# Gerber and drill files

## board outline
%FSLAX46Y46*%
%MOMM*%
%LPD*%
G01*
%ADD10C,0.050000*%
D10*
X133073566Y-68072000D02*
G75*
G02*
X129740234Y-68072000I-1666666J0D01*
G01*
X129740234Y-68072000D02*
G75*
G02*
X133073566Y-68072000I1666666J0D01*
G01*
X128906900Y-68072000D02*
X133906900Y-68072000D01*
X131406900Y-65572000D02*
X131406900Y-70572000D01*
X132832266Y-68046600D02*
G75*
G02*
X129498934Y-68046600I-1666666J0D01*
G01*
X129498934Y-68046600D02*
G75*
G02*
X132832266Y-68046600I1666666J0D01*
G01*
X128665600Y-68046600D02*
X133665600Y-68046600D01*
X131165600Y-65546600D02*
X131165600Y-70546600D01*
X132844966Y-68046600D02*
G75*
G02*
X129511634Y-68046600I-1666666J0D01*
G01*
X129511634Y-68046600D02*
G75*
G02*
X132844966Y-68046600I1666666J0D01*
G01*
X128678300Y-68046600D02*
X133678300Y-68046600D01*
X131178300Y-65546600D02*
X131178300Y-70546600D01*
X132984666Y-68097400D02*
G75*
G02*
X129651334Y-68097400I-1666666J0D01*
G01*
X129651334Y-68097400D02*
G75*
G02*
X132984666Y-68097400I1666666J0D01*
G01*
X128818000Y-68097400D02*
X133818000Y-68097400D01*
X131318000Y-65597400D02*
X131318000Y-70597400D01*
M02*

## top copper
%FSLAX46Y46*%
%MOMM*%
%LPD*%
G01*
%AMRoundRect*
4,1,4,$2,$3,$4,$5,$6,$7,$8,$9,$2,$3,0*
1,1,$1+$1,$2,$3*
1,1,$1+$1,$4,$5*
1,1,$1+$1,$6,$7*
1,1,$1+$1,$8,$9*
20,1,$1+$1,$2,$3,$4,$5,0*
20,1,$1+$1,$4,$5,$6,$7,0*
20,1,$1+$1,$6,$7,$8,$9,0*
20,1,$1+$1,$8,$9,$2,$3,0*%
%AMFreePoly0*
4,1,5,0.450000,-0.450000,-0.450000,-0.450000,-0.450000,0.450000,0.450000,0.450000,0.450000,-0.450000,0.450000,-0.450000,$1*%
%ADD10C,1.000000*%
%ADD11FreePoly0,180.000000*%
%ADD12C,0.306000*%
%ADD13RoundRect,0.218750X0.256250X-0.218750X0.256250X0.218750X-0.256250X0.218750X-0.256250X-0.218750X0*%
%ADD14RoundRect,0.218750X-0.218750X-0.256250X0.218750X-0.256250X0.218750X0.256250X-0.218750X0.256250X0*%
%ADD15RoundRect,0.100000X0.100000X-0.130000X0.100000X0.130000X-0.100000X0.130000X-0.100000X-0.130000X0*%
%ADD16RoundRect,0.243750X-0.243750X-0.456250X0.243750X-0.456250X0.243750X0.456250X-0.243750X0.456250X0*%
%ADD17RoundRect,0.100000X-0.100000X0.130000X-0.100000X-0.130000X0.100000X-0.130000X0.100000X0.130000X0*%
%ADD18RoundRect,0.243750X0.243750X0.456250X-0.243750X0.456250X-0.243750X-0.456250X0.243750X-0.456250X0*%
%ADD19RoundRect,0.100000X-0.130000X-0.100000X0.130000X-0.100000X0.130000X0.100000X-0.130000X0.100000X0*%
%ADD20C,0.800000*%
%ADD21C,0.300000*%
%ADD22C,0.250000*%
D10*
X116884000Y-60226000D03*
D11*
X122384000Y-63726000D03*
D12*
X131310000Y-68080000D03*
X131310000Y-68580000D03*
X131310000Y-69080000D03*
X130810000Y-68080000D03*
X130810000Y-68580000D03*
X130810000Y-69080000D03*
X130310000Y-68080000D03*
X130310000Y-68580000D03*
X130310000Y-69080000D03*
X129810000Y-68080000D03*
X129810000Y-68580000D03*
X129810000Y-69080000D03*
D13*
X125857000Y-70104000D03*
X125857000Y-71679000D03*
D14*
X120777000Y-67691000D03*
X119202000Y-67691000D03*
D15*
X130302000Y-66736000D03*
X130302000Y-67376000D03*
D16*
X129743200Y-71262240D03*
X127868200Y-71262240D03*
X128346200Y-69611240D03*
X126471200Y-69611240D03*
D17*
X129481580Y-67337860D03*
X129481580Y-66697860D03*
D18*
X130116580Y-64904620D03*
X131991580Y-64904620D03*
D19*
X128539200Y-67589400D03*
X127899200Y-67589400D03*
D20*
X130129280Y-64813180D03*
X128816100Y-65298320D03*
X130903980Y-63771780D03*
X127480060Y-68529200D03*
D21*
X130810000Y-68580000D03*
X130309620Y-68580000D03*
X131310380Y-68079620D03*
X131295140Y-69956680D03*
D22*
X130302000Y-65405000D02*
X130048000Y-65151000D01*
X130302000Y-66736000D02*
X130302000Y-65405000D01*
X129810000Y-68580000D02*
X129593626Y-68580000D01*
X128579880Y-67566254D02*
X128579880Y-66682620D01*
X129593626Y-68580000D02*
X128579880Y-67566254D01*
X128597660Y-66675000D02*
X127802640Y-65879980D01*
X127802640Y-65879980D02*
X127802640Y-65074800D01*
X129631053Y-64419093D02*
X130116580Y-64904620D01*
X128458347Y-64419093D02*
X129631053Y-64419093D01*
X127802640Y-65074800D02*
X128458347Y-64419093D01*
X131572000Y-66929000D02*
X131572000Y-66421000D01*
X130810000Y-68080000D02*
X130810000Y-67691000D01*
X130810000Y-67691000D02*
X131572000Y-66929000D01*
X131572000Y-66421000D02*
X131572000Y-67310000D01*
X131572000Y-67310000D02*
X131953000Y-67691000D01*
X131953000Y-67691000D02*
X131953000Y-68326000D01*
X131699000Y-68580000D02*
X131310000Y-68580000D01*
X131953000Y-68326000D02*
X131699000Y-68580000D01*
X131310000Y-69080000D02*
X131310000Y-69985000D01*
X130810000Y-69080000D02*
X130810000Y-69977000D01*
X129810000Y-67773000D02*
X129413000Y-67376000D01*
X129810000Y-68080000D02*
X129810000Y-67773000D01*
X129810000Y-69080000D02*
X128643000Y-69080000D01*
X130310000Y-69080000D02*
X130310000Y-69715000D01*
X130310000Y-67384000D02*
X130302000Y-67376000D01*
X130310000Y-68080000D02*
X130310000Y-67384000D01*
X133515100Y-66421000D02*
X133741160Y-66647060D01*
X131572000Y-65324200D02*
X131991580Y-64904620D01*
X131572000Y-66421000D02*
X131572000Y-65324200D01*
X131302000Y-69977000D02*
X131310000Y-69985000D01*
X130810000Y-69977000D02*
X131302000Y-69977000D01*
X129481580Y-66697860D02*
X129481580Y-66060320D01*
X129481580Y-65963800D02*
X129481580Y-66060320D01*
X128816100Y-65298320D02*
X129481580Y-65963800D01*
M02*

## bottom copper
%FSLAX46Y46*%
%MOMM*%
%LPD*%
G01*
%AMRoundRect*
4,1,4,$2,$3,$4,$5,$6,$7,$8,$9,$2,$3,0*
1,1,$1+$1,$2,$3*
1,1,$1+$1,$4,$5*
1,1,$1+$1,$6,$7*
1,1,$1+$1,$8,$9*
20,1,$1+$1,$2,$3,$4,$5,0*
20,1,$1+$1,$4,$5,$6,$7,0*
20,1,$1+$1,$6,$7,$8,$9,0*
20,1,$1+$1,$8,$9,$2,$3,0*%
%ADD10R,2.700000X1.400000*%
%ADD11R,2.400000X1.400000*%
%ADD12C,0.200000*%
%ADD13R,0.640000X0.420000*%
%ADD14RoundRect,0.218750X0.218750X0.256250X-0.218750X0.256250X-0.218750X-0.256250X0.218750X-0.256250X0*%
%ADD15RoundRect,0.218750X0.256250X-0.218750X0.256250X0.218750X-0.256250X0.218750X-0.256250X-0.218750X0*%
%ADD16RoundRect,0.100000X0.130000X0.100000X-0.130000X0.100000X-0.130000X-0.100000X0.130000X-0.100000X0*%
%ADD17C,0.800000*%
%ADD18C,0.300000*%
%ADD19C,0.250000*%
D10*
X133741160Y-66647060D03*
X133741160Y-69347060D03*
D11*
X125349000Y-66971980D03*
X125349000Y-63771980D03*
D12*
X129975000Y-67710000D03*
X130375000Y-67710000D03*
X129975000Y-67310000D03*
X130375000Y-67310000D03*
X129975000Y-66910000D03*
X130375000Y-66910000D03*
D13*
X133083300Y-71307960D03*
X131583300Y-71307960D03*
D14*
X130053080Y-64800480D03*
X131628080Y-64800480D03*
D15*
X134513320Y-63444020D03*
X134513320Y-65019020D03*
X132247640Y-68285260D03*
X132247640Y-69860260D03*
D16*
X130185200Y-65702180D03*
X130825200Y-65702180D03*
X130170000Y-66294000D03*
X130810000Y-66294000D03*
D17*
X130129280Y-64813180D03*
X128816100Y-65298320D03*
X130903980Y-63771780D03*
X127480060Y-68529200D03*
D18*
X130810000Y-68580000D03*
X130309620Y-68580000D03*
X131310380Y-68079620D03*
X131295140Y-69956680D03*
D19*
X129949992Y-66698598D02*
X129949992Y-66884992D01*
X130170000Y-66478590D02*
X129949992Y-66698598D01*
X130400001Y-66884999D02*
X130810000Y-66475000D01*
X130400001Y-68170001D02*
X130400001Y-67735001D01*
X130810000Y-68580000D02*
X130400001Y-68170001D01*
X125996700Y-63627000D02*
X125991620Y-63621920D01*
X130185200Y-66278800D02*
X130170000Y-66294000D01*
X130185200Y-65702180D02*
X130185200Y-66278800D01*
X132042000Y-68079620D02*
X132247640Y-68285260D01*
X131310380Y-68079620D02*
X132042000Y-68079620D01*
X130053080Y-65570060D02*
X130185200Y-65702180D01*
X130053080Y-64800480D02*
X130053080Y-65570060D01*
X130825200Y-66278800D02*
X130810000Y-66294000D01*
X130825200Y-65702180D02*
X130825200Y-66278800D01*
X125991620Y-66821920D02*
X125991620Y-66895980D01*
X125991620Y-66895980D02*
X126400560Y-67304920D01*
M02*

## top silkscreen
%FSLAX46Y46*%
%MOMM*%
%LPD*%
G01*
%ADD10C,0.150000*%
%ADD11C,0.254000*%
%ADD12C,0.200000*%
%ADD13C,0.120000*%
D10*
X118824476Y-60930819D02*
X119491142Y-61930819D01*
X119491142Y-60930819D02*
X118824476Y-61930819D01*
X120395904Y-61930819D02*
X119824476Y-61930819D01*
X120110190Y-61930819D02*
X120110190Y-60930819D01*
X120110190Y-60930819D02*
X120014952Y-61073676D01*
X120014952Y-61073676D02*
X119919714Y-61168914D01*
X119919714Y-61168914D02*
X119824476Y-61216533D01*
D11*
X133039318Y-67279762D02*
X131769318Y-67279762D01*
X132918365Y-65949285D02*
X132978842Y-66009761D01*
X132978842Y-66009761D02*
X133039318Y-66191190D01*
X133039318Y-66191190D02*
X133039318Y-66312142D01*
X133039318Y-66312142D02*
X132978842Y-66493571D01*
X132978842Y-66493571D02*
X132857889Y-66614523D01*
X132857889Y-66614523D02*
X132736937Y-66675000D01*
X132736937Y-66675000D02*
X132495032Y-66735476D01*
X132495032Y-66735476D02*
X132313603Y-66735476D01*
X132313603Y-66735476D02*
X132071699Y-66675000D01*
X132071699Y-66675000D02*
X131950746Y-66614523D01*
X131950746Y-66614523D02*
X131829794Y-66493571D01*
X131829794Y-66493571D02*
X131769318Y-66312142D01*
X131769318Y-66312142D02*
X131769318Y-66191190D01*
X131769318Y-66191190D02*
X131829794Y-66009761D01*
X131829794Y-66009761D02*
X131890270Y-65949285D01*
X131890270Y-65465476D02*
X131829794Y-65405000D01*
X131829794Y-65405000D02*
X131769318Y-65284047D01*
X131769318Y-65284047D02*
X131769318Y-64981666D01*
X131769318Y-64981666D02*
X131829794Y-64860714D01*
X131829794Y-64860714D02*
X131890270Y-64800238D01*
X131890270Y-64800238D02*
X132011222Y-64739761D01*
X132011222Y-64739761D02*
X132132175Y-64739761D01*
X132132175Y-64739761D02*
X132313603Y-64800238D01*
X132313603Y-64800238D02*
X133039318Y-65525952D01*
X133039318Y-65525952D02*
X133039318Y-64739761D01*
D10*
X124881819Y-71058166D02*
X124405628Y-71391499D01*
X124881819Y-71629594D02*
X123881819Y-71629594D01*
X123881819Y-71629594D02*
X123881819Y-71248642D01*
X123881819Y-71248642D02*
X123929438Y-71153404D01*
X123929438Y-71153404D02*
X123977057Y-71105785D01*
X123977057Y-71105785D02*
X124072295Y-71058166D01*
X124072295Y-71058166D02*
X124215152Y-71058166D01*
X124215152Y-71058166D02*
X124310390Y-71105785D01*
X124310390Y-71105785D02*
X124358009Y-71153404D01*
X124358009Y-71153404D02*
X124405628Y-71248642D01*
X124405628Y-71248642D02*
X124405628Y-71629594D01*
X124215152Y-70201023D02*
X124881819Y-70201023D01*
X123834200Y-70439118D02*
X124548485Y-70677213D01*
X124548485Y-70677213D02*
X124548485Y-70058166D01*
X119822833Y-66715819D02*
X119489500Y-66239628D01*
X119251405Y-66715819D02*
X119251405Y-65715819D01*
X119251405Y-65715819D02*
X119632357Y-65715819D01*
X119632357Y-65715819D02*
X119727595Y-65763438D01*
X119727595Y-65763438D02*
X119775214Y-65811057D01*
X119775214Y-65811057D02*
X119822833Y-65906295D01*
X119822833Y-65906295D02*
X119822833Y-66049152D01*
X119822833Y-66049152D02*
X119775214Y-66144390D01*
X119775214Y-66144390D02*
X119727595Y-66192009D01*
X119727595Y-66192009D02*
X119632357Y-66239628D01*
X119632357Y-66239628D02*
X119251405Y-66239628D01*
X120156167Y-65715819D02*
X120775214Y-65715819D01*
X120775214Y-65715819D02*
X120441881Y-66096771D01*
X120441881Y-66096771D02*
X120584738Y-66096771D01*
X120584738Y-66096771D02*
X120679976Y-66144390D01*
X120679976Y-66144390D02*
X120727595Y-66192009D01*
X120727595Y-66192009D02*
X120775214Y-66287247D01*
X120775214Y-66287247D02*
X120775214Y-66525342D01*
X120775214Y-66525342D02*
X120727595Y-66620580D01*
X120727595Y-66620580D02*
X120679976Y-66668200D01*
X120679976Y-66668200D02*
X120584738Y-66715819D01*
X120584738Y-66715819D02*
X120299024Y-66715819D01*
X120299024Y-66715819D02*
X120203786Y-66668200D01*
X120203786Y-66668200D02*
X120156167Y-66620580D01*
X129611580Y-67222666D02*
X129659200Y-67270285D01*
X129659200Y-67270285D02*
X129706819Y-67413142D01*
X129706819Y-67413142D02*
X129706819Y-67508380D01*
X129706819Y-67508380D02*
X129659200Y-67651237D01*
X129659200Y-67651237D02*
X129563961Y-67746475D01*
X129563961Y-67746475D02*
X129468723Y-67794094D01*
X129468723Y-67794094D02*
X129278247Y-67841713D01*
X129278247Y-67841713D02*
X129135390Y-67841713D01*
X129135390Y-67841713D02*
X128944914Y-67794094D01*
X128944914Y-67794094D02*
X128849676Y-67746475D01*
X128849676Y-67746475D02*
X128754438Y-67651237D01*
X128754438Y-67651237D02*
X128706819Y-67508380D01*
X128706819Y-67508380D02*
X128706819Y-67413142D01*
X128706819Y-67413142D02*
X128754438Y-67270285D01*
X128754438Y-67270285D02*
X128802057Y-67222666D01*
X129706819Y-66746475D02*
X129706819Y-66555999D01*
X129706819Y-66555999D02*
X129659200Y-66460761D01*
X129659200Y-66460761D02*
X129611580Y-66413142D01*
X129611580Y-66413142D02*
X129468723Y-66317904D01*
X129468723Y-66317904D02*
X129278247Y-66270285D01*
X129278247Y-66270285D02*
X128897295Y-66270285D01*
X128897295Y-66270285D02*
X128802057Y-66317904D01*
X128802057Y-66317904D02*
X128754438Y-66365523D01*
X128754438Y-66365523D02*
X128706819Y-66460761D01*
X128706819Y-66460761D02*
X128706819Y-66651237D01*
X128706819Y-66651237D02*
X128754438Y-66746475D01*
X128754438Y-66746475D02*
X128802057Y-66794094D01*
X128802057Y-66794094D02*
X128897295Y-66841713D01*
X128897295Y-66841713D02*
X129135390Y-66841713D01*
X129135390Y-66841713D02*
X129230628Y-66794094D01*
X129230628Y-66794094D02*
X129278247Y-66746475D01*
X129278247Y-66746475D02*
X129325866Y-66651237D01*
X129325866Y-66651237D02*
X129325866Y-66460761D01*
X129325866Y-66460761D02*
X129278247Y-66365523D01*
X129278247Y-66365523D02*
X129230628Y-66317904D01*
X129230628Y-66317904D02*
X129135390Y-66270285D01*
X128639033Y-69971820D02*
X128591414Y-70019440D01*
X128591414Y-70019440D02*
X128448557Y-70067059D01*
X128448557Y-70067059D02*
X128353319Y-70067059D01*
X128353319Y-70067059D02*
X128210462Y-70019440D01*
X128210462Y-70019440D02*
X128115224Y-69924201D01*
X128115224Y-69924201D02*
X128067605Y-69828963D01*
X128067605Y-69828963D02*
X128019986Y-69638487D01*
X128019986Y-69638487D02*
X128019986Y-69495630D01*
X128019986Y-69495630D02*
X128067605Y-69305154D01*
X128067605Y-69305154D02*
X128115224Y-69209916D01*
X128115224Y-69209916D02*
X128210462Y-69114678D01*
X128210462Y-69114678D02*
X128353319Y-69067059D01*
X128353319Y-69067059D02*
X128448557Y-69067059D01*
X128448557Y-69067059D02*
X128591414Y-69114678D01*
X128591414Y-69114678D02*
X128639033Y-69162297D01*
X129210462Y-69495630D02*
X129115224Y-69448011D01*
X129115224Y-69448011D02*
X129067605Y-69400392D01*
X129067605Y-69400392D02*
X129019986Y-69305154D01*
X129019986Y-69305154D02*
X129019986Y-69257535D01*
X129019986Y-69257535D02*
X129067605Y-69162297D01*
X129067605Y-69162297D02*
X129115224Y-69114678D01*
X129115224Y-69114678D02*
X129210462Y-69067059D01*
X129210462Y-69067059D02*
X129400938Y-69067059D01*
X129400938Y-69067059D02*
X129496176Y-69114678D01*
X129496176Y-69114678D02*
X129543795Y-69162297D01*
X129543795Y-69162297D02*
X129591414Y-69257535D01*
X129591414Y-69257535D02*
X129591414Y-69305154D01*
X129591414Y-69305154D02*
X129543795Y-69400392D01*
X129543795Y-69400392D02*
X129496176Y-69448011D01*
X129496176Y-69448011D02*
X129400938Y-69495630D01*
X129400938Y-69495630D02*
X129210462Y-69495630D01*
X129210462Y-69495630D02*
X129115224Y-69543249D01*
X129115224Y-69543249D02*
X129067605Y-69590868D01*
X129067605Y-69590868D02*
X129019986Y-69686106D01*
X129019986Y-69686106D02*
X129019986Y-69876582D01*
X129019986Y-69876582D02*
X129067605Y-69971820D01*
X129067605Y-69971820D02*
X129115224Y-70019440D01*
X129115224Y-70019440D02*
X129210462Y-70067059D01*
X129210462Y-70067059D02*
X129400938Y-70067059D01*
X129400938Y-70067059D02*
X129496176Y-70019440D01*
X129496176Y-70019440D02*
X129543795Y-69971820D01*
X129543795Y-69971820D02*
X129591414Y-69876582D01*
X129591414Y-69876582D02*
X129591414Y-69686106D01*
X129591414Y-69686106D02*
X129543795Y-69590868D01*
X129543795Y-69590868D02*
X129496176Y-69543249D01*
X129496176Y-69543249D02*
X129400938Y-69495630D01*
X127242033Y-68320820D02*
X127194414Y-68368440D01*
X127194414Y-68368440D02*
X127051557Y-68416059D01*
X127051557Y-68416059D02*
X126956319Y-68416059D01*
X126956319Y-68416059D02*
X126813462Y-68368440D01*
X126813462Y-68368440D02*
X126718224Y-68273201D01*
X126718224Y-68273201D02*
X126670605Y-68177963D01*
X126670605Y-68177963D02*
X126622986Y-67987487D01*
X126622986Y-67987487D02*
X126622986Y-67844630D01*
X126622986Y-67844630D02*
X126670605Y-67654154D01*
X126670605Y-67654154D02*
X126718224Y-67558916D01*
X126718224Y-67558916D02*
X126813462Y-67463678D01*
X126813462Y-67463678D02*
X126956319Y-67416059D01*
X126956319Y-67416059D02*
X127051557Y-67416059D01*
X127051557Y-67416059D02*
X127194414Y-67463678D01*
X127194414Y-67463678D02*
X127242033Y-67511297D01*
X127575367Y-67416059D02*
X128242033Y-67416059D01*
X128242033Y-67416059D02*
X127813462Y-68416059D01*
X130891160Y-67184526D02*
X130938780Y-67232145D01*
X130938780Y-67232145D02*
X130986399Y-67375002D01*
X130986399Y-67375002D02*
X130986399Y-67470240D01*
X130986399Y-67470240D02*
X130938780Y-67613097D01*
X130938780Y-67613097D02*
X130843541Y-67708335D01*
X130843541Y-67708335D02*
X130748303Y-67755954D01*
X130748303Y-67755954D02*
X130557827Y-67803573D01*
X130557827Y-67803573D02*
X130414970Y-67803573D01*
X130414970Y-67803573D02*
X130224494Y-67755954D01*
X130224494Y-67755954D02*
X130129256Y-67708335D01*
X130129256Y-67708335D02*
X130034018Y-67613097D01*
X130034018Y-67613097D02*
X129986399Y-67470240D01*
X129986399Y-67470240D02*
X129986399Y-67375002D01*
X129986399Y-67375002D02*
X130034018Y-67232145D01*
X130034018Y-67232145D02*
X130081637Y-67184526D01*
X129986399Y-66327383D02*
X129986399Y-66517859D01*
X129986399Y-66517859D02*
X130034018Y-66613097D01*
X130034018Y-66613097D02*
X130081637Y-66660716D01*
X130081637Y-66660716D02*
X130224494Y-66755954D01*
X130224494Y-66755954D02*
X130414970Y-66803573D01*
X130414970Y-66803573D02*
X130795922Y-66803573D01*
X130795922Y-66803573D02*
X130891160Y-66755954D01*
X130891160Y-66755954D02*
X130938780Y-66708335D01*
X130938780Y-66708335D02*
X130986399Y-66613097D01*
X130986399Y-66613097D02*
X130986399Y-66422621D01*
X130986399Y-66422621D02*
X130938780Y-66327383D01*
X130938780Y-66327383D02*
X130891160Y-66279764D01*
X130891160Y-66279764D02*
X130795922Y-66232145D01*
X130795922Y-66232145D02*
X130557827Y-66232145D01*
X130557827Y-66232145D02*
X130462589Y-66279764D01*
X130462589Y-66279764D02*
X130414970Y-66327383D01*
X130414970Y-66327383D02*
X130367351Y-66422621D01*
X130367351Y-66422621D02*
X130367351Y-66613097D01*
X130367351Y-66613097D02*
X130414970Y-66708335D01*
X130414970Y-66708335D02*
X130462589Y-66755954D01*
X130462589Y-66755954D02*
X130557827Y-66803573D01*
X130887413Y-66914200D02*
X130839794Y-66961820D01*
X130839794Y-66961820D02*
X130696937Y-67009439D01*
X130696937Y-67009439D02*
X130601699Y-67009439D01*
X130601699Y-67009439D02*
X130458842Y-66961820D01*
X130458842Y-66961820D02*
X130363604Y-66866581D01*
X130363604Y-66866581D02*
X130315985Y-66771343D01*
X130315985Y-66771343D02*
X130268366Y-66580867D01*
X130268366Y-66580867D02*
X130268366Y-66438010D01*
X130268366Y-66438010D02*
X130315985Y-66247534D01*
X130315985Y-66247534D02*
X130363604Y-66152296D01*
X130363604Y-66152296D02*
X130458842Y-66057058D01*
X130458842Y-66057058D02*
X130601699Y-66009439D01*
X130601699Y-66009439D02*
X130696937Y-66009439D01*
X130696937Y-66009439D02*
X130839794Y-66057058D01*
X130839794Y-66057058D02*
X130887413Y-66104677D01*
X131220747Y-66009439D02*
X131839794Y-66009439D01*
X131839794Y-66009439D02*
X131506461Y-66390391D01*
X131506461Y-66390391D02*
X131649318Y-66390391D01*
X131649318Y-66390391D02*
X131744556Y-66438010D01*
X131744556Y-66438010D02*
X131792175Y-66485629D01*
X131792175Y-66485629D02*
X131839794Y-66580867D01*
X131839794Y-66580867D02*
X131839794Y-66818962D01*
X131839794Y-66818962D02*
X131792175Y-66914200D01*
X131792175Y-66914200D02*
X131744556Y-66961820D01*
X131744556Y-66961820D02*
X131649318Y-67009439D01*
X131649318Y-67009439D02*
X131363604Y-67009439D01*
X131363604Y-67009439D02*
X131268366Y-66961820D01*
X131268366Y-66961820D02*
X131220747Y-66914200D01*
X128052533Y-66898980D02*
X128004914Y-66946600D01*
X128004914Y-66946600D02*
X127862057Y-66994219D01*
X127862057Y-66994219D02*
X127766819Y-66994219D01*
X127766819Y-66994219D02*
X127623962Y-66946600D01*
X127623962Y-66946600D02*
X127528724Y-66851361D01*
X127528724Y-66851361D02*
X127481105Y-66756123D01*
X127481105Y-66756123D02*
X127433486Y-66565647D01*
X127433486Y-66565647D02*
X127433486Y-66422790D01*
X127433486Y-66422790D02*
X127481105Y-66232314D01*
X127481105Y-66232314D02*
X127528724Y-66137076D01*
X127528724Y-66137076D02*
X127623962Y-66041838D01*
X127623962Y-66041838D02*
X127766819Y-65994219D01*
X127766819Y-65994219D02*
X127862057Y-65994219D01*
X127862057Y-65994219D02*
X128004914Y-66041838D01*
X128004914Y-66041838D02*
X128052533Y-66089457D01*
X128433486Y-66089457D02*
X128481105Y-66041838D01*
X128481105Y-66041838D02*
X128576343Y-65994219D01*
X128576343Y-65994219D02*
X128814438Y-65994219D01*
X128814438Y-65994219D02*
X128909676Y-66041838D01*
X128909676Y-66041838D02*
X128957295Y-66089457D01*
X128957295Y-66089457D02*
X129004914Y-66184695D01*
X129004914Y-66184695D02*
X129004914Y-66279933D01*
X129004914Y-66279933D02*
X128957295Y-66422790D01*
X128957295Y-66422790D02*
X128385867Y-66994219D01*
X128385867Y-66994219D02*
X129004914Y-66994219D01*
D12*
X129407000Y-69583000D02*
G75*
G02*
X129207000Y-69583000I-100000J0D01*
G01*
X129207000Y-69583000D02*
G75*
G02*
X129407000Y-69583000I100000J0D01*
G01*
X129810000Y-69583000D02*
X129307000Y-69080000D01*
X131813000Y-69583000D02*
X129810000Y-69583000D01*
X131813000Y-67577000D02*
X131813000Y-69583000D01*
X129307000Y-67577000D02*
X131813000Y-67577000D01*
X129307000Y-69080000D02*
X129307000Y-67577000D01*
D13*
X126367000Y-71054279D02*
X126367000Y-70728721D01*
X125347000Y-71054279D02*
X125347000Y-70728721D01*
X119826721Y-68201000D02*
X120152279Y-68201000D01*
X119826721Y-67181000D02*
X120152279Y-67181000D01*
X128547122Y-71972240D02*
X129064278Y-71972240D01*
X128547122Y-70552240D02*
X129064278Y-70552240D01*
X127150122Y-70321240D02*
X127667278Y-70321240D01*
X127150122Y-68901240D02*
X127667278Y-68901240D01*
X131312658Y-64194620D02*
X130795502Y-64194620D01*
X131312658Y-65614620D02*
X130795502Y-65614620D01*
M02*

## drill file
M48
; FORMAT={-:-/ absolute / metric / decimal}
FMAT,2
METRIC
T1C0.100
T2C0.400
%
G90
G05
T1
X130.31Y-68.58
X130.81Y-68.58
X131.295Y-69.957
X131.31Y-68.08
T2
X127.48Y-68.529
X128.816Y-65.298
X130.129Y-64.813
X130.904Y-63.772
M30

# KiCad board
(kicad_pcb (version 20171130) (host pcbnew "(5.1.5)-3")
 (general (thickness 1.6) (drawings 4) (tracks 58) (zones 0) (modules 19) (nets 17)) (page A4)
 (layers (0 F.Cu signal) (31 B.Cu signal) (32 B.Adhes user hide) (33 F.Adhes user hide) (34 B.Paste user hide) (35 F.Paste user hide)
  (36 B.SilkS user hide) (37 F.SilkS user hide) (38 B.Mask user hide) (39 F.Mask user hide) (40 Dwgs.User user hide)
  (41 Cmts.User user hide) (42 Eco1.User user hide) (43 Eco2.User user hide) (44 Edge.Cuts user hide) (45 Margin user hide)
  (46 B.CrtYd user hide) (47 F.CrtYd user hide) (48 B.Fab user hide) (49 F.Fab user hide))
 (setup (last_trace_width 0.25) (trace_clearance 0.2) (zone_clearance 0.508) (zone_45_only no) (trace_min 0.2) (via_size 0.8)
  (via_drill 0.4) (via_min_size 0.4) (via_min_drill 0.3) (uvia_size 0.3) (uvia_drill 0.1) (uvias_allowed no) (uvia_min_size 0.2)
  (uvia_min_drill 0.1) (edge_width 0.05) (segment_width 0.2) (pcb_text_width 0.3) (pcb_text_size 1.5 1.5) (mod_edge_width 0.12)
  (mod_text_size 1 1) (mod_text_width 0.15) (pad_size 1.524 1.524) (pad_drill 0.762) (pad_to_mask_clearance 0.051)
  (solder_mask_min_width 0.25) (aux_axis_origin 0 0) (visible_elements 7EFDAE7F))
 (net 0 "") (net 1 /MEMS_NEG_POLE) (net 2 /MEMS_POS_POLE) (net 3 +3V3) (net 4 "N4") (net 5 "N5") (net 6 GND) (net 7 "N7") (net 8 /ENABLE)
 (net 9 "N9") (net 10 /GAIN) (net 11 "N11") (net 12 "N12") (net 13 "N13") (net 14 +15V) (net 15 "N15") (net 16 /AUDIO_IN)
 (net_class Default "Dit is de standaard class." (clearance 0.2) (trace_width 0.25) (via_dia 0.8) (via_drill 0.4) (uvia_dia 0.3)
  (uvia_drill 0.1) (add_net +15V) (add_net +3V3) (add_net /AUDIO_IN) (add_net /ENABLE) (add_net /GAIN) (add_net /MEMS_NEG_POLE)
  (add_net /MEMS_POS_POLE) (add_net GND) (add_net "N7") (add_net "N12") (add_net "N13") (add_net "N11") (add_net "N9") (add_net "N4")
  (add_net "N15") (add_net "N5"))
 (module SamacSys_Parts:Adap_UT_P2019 (layer F.Cu) (at 119.634 61.976 180) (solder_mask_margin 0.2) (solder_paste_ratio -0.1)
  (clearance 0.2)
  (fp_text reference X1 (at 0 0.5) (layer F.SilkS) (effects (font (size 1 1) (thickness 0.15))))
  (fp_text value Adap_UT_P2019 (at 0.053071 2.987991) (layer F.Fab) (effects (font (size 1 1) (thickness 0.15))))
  (pad 2 smd circle (at 2.75 1.75 180) (size 1 1) (layers F.Cu F.Paste F.Mask) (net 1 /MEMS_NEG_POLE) (zone_connect 0))
  (pad 1 smd custom (at -2.75 -1.75 180) (size 0.9 0.9) (layers F.Cu F.Paste F.Mask) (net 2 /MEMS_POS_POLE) (zone_connect 0)
   (options (clearance outline) (anchor rect)) (primitives)))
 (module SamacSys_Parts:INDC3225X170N (layer B.Cu) (at 133.74116 67.99706 90)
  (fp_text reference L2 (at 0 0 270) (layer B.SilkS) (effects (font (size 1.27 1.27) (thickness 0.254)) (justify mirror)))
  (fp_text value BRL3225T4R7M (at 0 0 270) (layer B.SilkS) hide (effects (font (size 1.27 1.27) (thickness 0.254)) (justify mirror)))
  (pad 2 smd rect (at 1.35 0 90) (size 1.4 2.7) (layers B.Cu B.Paste B.Mask) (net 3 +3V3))
  (pad 1 smd rect (at -1.35 0 90) (size 1.4 2.7) (layers B.Cu B.Paste B.Mask) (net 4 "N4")))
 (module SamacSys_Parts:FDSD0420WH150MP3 (layer B.Cu) (at 125.349 65.37198 270)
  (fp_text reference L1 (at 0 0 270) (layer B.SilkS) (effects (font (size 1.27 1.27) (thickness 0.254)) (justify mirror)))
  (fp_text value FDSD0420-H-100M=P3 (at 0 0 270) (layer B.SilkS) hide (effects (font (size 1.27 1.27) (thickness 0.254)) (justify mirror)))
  (pad 2 smd rect (at 1.6 0 270) (size 1.4 2.4) (layers B.Cu B.Paste B.Mask) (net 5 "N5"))
  (pad 1 smd rect (at -1.6 0 270) (size 1.4 2.4) (layers B.Cu B.Paste B.Mask) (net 3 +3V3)))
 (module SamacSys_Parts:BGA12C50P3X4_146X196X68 (layer F.Cu) (at 130.56 68.58 90)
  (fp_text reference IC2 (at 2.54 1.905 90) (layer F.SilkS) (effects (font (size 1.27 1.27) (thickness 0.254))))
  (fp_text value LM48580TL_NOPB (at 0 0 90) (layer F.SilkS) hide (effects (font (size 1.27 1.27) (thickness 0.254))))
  (fp_circle (center -1.003 -1.253) (end -1.003 -1.153) (layer F.SilkS) (width 0.2))
  (fp_line (start -1.003 -0.75) (end -0.5 -1.253) (layer F.SilkS) (width 0.2))
  (fp_line (start -1.003 1.253) (end -1.003 -0.75) (layer F.SilkS) (width 0.2))
  (fp_line (start 1.003 1.253) (end -1.003 1.253) (layer F.SilkS) (width 0.2))
  (fp_line (start 1.003 -1.253) (end 1.003 1.253) (layer F.SilkS) (width 0.2))
  (fp_line (start -0.5 -1.253) (end 1.003 -1.253) (layer F.SilkS) (width 0.2))
  (pad D3 smd circle (at 0.5 0.75 180) (size 0.306 0.306) (layers F.Cu F.Paste F.Mask) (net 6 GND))
  (pad D2 smd circle (at 0 0.75 180) (size 0.306 0.306) (layers F.Cu F.Paste F.Mask) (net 3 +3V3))
  (pad D1 smd circle (at -0.5 0.75 180) (size 0.306 0.306) (layers F.Cu F.Paste F.Mask) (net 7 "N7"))
  (pad C3 smd circle (at 0.5 0.25 180) (size 0.306 0.306) (layers F.Cu F.Paste F.Mask) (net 3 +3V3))
  (pad C2 smd circle (at 0 0.25 180) (size 0.306 0.306) (layers F.Cu F.Paste F.Mask) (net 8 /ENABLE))
  (pad C1 smd circle (at -0.5 0.25 180) (size 0.306 0.306) (layers F.Cu F.Paste F.Mask) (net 7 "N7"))
  (pad B3 smd circle (at 0.5 -0.25 180) (size 0.306 0.306) (layers F.Cu F.Paste F.Mask) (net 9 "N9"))
  (pad B2 smd circle (at 0 -0.25 180) (size 0.306 0.306) (layers F.Cu F.Paste F.Mask) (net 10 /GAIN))
  (pad B1 smd circle (at -0.5 -0.25 180) (size 0.306 0.306) (layers F.Cu F.Paste F.Mask) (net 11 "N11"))
  (pad A3 smd circle (at 0.5 -0.75 180) (size 0.306 0.306) (layers F.Cu F.Paste F.Mask) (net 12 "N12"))
  (pad A2 smd circle (at 0 -0.75 180) (size 0.306 0.306) (layers F.Cu F.Paste F.Mask) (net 6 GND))
  (pad A1 smd circle (at -0.5 -0.75 180) (size 0.306 0.306) (layers F.Cu F.Paste F.Mask) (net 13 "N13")))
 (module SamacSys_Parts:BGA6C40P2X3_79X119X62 (layer B.Cu) (at 130.175 67.31 180)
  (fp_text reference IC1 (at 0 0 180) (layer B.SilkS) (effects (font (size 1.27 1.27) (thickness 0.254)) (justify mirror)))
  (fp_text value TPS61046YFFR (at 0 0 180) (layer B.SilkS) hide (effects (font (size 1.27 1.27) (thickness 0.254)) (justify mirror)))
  (pad C2 smd circle (at 0.2 -0.4 90) (size 0.2 0.2) (layers B.Cu B.Paste B.Mask) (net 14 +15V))
  (pad C1 smd circle (at -0.2 -0.4 90) (size 0.2 0.2) (layers B.Cu B.Paste B.Mask) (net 8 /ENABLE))
  (pad B2 smd circle (at 0.2 0 90) (size 0.2 0.2) (layers B.Cu B.Paste B.Mask) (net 5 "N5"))
  (pad B1 smd circle (at -0.2 0 90) (size 0.2 0.2) (layers B.Cu B.Paste B.Mask) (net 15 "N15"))
  (pad A2 smd circle (at 0.2 0.4 90) (size 0.2 0.2) (layers B.Cu B.Paste B.Mask) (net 6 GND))
  (pad A1 smd circle (at -0.2 0.4 90) (size 0.2 0.2) (layers B.Cu B.Paste B.Mask) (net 3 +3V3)))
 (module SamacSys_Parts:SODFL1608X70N (layer B.Cu) (at 132.3333 71.30796)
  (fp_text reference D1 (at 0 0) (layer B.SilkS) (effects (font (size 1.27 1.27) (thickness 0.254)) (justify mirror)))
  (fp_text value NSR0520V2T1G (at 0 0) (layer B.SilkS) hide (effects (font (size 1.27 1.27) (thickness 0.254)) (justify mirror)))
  (pad 2 smd rect (at 0.75 0 270) (size 0.42 0.64) (layers B.Cu B.Paste B.Mask) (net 4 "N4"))
  (pad 1 smd rect (at -0.75 0 270) (size 0.42 0.64) (layers B.Cu B.Paste B.Mask) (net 7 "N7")))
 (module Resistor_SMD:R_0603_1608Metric (layer F.Cu) (at 125.857 70.8915 90)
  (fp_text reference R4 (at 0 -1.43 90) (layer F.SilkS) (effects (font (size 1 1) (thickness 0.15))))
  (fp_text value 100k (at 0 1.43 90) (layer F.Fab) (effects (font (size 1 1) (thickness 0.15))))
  (fp_line (start -0.162779 0.51) (end 0.162779 0.51) (layer F.SilkS) (width 0.12))
  (fp_line (start -0.162779 -0.51) (end 0.162779 -0.51) (layer F.SilkS) (width 0.12))
  (pad 2 smd roundrect (at 0.7875 0 90) (size 0.875 0.95) (layers F.Cu F.Paste F.Mask) (roundrect_rratio 0.25) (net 14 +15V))
  (pad 1 smd roundrect (at -0.7875 0 90) (size 0.875 0.95) (layers F.Cu F.Paste F.Mask) (roundrect_rratio 0.25) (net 1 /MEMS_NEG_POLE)))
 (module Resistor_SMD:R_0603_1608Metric (layer F.Cu) (at 119.9895 67.691)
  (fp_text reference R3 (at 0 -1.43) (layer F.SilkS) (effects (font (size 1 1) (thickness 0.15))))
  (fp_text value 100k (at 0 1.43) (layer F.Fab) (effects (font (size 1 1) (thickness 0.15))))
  (fp_line (start -0.162779 0.51) (end 0.162779 0.51) (layer F.SilkS) (width 0.12))
  (fp_line (start -0.162779 -0.51) (end 0.162779 -0.51) (layer F.SilkS) (width 0.12))
  (pad 2 smd roundrect (at 0.7875 0) (size 0.875 0.95) (layers F.Cu F.Paste F.Mask) (roundrect_rratio 0.25) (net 14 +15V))
  (pad 1 smd roundrect (at -0.7875 0) (size 0.875 0.95) (layers F.Cu F.Paste F.Mask) (roundrect_rratio 0.25) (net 2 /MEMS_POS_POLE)))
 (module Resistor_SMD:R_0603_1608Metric (layer B.Cu) (at 130.84058 64.80048 180)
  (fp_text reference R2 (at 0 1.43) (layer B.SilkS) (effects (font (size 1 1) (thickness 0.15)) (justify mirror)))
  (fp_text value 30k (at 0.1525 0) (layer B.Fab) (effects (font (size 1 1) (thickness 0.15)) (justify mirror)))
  (pad 2 smd roundrect (at 0.7875 0 180) (size 0.875 0.95) (layers B.Cu B.Paste B.Mask) (roundrect_rratio 0.25) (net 6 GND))
  (pad 1 smd roundrect (at -0.7875 0 180) (size 0.875 0.95) (layers B.Cu B.Paste B.Mask) (roundrect_rratio 0.25) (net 15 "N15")))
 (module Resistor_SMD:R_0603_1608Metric (layer B.Cu) (at 134.51332 64.23152 90)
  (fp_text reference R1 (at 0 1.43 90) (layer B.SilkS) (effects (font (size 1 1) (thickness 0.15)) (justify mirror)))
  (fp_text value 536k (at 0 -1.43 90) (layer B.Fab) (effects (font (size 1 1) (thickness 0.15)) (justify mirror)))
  (pad 2 smd roundrect (at 0.7875 0 90) (size 0.875 0.95) (layers B.Cu B.Paste B.Mask) (roundrect_rratio 0.25) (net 15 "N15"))
  (pad 1 smd roundrect (at -0.7875 0 90) (size 0.875 0.95) (layers B.Cu B.Paste B.Mask) (roundrect_rratio 0.25) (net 14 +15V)))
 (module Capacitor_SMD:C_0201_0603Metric (layer F.Cu) (at 130.302 67.056 90)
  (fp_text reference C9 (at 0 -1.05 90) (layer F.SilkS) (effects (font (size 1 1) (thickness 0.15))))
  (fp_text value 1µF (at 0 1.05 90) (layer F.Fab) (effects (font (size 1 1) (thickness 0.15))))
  (pad 2 smd roundrect (at 0.32 0 90) (size 0.46 0.4) (layers F.Cu F.Mask) (roundrect_rratio 0.25) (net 6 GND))
  (pad 1 smd roundrect (at -0.32 0 90) (size 0.46 0.4) (layers F.Cu F.Mask) (roundrect_rratio 0.25) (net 9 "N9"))
  (pad "" smd roundrect (at 0.345 0 90) (size 0.318 0.36) (layers F.Paste) (roundrect_rratio 0.25))
  (pad "" smd roundrect (at -0.345 0 90) (size 0.318 0.36) (layers F.Paste) (roundrect_rratio 0.25)))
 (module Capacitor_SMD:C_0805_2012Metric (layer F.Cu) (at 128.8057 71.26224)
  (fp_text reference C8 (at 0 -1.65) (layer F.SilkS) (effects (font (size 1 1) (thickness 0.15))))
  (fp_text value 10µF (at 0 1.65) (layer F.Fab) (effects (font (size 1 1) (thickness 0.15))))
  (fp_line (start -0.258578 0.71) (end 0.258578 0.71) (layer F.SilkS) (width 0.12))
  (fp_line (start -0.258578 -0.71) (end 0.258578 -0.71) (layer F.SilkS) (width 0.12))
  (pad 2 smd roundrect (at 0.9375 0) (size 0.975 1.4) (layers F.Cu F.Paste F.Mask) (roundrect_rratio 0.25) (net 11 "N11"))
  (pad 1 smd roundrect (at -0.9375 0) (size 0.975 1.4) (layers F.Cu F.Paste F.Mask) (roundrect_rratio 0.25) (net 1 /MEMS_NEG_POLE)))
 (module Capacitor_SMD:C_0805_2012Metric (layer F.Cu) (at 127.4087 69.61124)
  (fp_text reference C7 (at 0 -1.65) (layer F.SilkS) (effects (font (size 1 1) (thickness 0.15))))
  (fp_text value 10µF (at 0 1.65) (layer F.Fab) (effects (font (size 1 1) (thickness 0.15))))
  (fp_line (start -0.258578 0.71) (end 0.258578 0.71) (layer F.SilkS) (width 0.12))
  (fp_line (start -0.258578 -0.71) (end 0.258578 -0.71) (layer F.SilkS) (width 0.12))
  (pad 2 smd roundrect (at 0.9375 0) (size 0.975 1.4) (layers F.Cu F.Paste F.Mask) (roundrect_rratio 0.25) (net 13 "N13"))
  (pad 1 smd roundrect (at -0.9375 0) (size 0.975 1.4) (layers F.Cu F.Paste F.Mask) (roundrect_rratio 0.25) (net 2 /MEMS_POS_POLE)))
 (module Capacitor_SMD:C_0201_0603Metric (layer F.Cu) (at 129.48158 67.01786 270)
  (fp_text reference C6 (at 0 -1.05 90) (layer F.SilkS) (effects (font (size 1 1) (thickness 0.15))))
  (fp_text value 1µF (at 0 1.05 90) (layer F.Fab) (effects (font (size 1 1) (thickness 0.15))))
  (pad 2 smd roundrect (at 0.32 0 270) (size 0.46 0.4) (layers F.Cu F.Mask) (roundrect_rratio 0.25) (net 12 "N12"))
  (pad 1 smd roundrect (at -0.32 0 270) (size 0.46 0.4) (layers F.Cu F.Mask) (roundrect_rratio 0.25) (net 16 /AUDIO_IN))
  (pad "" smd roundrect (at 0.345 0 270) (size 0.318 0.36) (layers F.Paste) (roundrect_rratio 0.25))
  (pad "" smd roundrect (at -0.345 0 270) (size 0.318 0.36) (layers F.Paste) (roundrect_rratio 0.25)))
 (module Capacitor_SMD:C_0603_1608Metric (layer B.Cu) (at 132.24764 69.07276 90)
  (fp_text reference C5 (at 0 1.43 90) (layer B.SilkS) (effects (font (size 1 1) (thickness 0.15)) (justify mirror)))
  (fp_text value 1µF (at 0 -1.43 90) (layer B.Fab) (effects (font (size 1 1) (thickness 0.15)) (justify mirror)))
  (pad 2 smd roundrect (at 0.7875 0 90) (size 0.875 0.95) (layers B.Cu B.Paste B.Mask) (roundrect_rratio 0.25) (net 6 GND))
  (pad 1 smd roundrect (at -0.7875 0 90) (size 0.875 0.95) (layers B.Cu B.Paste B.Mask) (roundrect_rratio 0.25) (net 7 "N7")))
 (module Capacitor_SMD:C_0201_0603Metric (layer B.Cu) (at 130.5052 65.70218 180)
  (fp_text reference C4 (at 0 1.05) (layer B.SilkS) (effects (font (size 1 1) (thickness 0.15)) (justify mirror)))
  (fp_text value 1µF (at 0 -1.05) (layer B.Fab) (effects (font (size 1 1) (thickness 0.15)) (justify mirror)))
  (pad 2 smd roundrect (at 0.32 0 180) (size 0.46 0.4) (layers B.Cu B.Mask) (roundrect_rratio 0.25) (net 6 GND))
  (pad 1 smd roundrect (at -0.32 0 180) (size 0.46 0.4) (layers B.Cu B.Mask) (roundrect_rratio 0.25) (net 3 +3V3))
  (pad "" smd roundrect (at 0.345 0 180) (size 0.318 0.36) (layers B.Paste) (roundrect_rratio 0.25))
  (pad "" smd roundrect (at -0.345 0 180) (size 0.318 0.36) (layers B.Paste) (roundrect_rratio 0.25)))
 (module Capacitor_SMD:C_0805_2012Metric (layer F.Cu) (at 131.05408 64.90462 180)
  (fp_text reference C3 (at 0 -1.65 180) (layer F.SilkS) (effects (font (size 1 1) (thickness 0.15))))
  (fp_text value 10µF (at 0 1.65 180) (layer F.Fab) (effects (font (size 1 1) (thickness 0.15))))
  (fp_line (start -0.258578 0.71) (end 0.258578 0.71) (layer F.SilkS) (width 0.12))
  (fp_line (start -0.258578 -0.71) (end 0.258578 -0.71) (layer F.SilkS) (width 0.12))
  (pad 2 smd roundrect (at 0.9375 0 180) (size 0.975 1.4) (layers F.Cu F.Paste F.Mask) (roundrect_rratio 0.25) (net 6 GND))
  (pad 1 smd roundrect (at -0.9375 0 180) (size 0.975 1.4) (layers F.Cu F.Paste F.Mask) (roundrect_rratio 0.25) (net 3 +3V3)))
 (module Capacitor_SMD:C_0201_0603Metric (layer F.Cu) (at 128.2192 67.5894)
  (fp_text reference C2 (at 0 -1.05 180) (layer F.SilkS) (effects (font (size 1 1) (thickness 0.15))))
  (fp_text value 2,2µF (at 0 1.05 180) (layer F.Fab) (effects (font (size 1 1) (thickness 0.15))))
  (pad 2 smd roundrect (at 0.32 0) (size 0.46 0.4) (layers F.Cu F.Mask) (roundrect_rratio 0.25) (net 6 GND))
  (pad 1 smd roundrect (at -0.32 0) (size 0.46 0.4) (layers F.Cu F.Mask) (roundrect_rratio 0.25) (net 14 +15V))
  (pad "" smd roundrect (at 0.345 0) (size 0.318 0.36) (layers F.Paste) (roundrect_rratio 0.25))
  (pad "" smd roundrect (at -0.345 0) (size 0.318 0.36) (layers F.Paste) (roundrect_rratio 0.25)))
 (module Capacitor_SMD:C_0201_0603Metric (layer B.Cu) (at 130.49 66.294 180)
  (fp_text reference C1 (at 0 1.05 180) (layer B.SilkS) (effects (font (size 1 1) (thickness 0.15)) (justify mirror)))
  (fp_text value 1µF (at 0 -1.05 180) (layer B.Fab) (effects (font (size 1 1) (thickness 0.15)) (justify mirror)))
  (pad 2 smd roundrect (at 0.32 0 180) (size 0.46 0.4) (layers B.Cu B.Mask) (roundrect_rratio 0.25) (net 6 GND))
  (pad 1 smd roundrect (at -0.32 0 180) (size 0.46 0.4) (layers B.Cu B.Mask) (roundrect_rratio 0.25) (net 3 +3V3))
  (pad "" smd roundrect (at 0.345 0 180) (size 0.318 0.36) (layers B.Paste) (roundrect_rratio 0.25))
  (pad "" smd roundrect (at -0.345 0 180) (size 0.318 0.36) (layers B.Paste) (roundrect_rratio 0.25)))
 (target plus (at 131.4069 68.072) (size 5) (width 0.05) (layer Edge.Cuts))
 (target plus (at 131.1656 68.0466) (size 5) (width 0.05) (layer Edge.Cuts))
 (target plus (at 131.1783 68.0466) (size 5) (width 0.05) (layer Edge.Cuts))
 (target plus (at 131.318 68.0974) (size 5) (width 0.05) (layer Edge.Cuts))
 (via (at 130.12928 64.81318) (size 0.8) (drill 0.4) (layers F.Cu B.Cu) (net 6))
 (segment (start 130.302 65.405) (end 130.048 65.151) (width 0.25) (layer F.Cu) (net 6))
 (segment (start 130.302 66.736) (end 130.302 65.405) (width 0.25) (layer F.Cu) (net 6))
 (segment (start 129.949992 66.698598) (end 129.949992 66.884992) (width 0.25) (layer B.Cu) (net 6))
 (segment (start 130.17 66.47859) (end 129.949992 66.698598) (width 0.25) (layer B.Cu) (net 6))
 (segment (start 129.81 68.58) (end 129.593626 68.58) (width 0.25) (layer F.Cu) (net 6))
 (segment (start 128.57988 67.566254) (end 128.57988 66.68262) (width 0.25) (layer F.Cu) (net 6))
 (segment (start 129.593626 68.58) (end 128.57988 67.566254) (width 0.25) (layer F.Cu) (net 6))
 (segment (start 128.59766 66.675) (end 127.80264 65.87998) (width 0.25) (layer F.Cu) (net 6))
 (segment (start 127.80264 65.87998) (end 127.80264 65.0748) (width 0.25) (layer F.Cu) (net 6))
 (segment (start 129.631053 64.419093) (end 130.11658 64.90462) (width 0.25) (layer F.Cu) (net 6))
 (segment (start 128.458347 64.419093) (end 129.631053 64.419093) (width 0.25) (layer F.Cu) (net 6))
 (segment (start 127.80264 65.0748) (end 128.458347 64.419093) (width 0.25) (layer F.Cu) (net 6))
 (via (at 128.8161 65.29832) (size 0.8) (drill 0.4) (layers F.Cu B.Cu) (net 16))
 (via (at 130.90398 63.77178) (size 0.8) (drill 0.4) (layers F.Cu B.Cu) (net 3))
 (segment (start 130.400001 66.884999) (end 130.81 66.475) (width 0.25) (layer B.Cu) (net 3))
 (segment (start 131.572 66.929) (end 131.572 66.421) (width 0.25) (layer F.Cu) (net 3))
 (segment (start 130.81 68.08) (end 130.81 67.691) (width 0.25) (layer F.Cu) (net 3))
 (segment (start 130.81 67.691) (end 131.572 66.929) (width 0.25) (layer F.Cu) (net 3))
 (segment (start 131.572 66.421) (end 131.572 67.31) (width 0.25) (layer F.Cu) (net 3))
 (segment (start 131.572 67.31) (end 131.953 67.691) (width 0.25) (layer F.Cu) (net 3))
 (segment (start 131.953 67.691) (end 131.953 68.326) (width 0.25) (layer F.Cu) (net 3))
 (segment (start 131.699 68.58) (end 131.31 68.58) (width 0.25) (layer F.Cu) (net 3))
 (segment (start 131.953 68.326) (end 131.699 68.58) (width 0.25) (layer F.Cu) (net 3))
 (via (at 127.48006 68.5292) (size 0.8) (drill 0.4) (layers F.Cu B.Cu) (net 14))
 (segment (start 131.31 69.08) (end 131.31 69.985) (width 0.25) (layer F.Cu) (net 7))
 (segment (start 130.81 69.08) (end 130.81 69.977) (width 0.25) (layer F.Cu) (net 7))
 (segment (start 129.81 67.773) (end 129.413 67.376) (width 0.25) (layer F.Cu) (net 12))
 (segment (start 129.81 68.08) (end 129.81 67.773) (width 0.25) (layer F.Cu) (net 12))
 (segment (start 129.81 69.08) (end 128.643 69.08) (width 0.25) (layer F.Cu) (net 13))
 (segment (start 130.31 69.08) (end 130.31 69.715) (width 0.25) (layer F.Cu) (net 11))
 (segment (start 130.31 67.384) (end 130.302 67.376) (width 0.25) (layer F.Cu) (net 9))
 (segment (start 130.31 68.08) (end 130.31 67.384) (width 0.25) (layer F.Cu) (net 9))
 (via (at 130.81 68.58) (size 0.3) (drill 0.1) (layers F.Cu B.Cu) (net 8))
 (segment (start 130.400001 68.170001) (end 130.400001 67.735001) (width 0.25) (layer B.Cu) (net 8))
 (segment (start 130.81 68.58) (end 130.400001 68.170001) (width 0.25) (layer B.Cu) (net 8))
 (via (at 130.30962 68.58) (size 0.3) (drill 0.1) (layers F.Cu B.Cu) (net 10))
 (segment (start 133.5151 66.421) (end 133.74116 66.64706) (width 0.25) (layer F.Cu) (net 3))
 (segment (start 131.572 65.3242) (end 131.99158 64.90462) (width 0.25) (layer F.Cu) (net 3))
 (segment (start 131.572 66.421) (end 131.572 65.3242) (width 0.25) (layer F.Cu) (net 3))
 (segment (start 125.9967 63.627) (end 125.99162 63.62192) (width 0.25) (layer B.Cu) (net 3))
 (segment (start 131.302 69.977) (end 131.31 69.985) (width 0.25) (layer F.Cu) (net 7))
 (segment (start 130.81 69.977) (end 131.302 69.977) (width 0.25) (layer F.Cu) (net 7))
 (segment (start 129.48158 66.69786) (end 129.48158 66.06032) (width 0.25) (layer F.Cu) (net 16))
 (segment (start 129.48158 65.9638) (end 129.48158 66.06032) (width 0.25) (layer F.Cu) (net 16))
 (segment (start 128.8161 65.29832) (end 129.48158 65.9638) (width 0.25) (layer F.Cu) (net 16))
 (via (at 131.31038 68.07962) (size 0.3) (drill 0.1) (layers F.Cu B.Cu) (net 6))
 (segment (start 130.1852 66.2788) (end 130.17 66.294) (width 0.25) (layer B.Cu) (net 6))
 (segment (start 130.1852 65.70218) (end 130.1852 66.2788) (width 0.25) (layer B.Cu) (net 6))
 (segment (start 132.042 68.07962) (end 132.24764 68.28526) (width 0.25) (layer B.Cu) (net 6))
 (segment (start 131.31038 68.07962) (end 132.042 68.07962) (width 0.25) (layer B.Cu) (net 6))
 (segment (start 130.05308 65.57006) (end 130.1852 65.70218) (width 0.25) (layer B.Cu) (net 6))
 (segment (start 130.05308 64.80048) (end 130.05308 65.57006) (width 0.25) (layer B.Cu) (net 6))
 (segment (start 130.8252 66.2788) (end 130.81 66.294) (width 0.25) (layer B.Cu) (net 3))
 (segment (start 130.8252 65.70218) (end 130.8252 66.2788) (width 0.25) (layer B.Cu) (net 3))
 (via (at 131.29514 69.95668) (size 0.3) (drill 0.1) (layers F.Cu B.Cu) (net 7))
 (segment (start 125.99162 66.82192) (end 125.99162 66.89598) (width 0.25) (layer B.Cu) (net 5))
 (segment (start 125.99162 66.89598) (end 126.40056 67.30492) (width 0.25) (layer B.Cu) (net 5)))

